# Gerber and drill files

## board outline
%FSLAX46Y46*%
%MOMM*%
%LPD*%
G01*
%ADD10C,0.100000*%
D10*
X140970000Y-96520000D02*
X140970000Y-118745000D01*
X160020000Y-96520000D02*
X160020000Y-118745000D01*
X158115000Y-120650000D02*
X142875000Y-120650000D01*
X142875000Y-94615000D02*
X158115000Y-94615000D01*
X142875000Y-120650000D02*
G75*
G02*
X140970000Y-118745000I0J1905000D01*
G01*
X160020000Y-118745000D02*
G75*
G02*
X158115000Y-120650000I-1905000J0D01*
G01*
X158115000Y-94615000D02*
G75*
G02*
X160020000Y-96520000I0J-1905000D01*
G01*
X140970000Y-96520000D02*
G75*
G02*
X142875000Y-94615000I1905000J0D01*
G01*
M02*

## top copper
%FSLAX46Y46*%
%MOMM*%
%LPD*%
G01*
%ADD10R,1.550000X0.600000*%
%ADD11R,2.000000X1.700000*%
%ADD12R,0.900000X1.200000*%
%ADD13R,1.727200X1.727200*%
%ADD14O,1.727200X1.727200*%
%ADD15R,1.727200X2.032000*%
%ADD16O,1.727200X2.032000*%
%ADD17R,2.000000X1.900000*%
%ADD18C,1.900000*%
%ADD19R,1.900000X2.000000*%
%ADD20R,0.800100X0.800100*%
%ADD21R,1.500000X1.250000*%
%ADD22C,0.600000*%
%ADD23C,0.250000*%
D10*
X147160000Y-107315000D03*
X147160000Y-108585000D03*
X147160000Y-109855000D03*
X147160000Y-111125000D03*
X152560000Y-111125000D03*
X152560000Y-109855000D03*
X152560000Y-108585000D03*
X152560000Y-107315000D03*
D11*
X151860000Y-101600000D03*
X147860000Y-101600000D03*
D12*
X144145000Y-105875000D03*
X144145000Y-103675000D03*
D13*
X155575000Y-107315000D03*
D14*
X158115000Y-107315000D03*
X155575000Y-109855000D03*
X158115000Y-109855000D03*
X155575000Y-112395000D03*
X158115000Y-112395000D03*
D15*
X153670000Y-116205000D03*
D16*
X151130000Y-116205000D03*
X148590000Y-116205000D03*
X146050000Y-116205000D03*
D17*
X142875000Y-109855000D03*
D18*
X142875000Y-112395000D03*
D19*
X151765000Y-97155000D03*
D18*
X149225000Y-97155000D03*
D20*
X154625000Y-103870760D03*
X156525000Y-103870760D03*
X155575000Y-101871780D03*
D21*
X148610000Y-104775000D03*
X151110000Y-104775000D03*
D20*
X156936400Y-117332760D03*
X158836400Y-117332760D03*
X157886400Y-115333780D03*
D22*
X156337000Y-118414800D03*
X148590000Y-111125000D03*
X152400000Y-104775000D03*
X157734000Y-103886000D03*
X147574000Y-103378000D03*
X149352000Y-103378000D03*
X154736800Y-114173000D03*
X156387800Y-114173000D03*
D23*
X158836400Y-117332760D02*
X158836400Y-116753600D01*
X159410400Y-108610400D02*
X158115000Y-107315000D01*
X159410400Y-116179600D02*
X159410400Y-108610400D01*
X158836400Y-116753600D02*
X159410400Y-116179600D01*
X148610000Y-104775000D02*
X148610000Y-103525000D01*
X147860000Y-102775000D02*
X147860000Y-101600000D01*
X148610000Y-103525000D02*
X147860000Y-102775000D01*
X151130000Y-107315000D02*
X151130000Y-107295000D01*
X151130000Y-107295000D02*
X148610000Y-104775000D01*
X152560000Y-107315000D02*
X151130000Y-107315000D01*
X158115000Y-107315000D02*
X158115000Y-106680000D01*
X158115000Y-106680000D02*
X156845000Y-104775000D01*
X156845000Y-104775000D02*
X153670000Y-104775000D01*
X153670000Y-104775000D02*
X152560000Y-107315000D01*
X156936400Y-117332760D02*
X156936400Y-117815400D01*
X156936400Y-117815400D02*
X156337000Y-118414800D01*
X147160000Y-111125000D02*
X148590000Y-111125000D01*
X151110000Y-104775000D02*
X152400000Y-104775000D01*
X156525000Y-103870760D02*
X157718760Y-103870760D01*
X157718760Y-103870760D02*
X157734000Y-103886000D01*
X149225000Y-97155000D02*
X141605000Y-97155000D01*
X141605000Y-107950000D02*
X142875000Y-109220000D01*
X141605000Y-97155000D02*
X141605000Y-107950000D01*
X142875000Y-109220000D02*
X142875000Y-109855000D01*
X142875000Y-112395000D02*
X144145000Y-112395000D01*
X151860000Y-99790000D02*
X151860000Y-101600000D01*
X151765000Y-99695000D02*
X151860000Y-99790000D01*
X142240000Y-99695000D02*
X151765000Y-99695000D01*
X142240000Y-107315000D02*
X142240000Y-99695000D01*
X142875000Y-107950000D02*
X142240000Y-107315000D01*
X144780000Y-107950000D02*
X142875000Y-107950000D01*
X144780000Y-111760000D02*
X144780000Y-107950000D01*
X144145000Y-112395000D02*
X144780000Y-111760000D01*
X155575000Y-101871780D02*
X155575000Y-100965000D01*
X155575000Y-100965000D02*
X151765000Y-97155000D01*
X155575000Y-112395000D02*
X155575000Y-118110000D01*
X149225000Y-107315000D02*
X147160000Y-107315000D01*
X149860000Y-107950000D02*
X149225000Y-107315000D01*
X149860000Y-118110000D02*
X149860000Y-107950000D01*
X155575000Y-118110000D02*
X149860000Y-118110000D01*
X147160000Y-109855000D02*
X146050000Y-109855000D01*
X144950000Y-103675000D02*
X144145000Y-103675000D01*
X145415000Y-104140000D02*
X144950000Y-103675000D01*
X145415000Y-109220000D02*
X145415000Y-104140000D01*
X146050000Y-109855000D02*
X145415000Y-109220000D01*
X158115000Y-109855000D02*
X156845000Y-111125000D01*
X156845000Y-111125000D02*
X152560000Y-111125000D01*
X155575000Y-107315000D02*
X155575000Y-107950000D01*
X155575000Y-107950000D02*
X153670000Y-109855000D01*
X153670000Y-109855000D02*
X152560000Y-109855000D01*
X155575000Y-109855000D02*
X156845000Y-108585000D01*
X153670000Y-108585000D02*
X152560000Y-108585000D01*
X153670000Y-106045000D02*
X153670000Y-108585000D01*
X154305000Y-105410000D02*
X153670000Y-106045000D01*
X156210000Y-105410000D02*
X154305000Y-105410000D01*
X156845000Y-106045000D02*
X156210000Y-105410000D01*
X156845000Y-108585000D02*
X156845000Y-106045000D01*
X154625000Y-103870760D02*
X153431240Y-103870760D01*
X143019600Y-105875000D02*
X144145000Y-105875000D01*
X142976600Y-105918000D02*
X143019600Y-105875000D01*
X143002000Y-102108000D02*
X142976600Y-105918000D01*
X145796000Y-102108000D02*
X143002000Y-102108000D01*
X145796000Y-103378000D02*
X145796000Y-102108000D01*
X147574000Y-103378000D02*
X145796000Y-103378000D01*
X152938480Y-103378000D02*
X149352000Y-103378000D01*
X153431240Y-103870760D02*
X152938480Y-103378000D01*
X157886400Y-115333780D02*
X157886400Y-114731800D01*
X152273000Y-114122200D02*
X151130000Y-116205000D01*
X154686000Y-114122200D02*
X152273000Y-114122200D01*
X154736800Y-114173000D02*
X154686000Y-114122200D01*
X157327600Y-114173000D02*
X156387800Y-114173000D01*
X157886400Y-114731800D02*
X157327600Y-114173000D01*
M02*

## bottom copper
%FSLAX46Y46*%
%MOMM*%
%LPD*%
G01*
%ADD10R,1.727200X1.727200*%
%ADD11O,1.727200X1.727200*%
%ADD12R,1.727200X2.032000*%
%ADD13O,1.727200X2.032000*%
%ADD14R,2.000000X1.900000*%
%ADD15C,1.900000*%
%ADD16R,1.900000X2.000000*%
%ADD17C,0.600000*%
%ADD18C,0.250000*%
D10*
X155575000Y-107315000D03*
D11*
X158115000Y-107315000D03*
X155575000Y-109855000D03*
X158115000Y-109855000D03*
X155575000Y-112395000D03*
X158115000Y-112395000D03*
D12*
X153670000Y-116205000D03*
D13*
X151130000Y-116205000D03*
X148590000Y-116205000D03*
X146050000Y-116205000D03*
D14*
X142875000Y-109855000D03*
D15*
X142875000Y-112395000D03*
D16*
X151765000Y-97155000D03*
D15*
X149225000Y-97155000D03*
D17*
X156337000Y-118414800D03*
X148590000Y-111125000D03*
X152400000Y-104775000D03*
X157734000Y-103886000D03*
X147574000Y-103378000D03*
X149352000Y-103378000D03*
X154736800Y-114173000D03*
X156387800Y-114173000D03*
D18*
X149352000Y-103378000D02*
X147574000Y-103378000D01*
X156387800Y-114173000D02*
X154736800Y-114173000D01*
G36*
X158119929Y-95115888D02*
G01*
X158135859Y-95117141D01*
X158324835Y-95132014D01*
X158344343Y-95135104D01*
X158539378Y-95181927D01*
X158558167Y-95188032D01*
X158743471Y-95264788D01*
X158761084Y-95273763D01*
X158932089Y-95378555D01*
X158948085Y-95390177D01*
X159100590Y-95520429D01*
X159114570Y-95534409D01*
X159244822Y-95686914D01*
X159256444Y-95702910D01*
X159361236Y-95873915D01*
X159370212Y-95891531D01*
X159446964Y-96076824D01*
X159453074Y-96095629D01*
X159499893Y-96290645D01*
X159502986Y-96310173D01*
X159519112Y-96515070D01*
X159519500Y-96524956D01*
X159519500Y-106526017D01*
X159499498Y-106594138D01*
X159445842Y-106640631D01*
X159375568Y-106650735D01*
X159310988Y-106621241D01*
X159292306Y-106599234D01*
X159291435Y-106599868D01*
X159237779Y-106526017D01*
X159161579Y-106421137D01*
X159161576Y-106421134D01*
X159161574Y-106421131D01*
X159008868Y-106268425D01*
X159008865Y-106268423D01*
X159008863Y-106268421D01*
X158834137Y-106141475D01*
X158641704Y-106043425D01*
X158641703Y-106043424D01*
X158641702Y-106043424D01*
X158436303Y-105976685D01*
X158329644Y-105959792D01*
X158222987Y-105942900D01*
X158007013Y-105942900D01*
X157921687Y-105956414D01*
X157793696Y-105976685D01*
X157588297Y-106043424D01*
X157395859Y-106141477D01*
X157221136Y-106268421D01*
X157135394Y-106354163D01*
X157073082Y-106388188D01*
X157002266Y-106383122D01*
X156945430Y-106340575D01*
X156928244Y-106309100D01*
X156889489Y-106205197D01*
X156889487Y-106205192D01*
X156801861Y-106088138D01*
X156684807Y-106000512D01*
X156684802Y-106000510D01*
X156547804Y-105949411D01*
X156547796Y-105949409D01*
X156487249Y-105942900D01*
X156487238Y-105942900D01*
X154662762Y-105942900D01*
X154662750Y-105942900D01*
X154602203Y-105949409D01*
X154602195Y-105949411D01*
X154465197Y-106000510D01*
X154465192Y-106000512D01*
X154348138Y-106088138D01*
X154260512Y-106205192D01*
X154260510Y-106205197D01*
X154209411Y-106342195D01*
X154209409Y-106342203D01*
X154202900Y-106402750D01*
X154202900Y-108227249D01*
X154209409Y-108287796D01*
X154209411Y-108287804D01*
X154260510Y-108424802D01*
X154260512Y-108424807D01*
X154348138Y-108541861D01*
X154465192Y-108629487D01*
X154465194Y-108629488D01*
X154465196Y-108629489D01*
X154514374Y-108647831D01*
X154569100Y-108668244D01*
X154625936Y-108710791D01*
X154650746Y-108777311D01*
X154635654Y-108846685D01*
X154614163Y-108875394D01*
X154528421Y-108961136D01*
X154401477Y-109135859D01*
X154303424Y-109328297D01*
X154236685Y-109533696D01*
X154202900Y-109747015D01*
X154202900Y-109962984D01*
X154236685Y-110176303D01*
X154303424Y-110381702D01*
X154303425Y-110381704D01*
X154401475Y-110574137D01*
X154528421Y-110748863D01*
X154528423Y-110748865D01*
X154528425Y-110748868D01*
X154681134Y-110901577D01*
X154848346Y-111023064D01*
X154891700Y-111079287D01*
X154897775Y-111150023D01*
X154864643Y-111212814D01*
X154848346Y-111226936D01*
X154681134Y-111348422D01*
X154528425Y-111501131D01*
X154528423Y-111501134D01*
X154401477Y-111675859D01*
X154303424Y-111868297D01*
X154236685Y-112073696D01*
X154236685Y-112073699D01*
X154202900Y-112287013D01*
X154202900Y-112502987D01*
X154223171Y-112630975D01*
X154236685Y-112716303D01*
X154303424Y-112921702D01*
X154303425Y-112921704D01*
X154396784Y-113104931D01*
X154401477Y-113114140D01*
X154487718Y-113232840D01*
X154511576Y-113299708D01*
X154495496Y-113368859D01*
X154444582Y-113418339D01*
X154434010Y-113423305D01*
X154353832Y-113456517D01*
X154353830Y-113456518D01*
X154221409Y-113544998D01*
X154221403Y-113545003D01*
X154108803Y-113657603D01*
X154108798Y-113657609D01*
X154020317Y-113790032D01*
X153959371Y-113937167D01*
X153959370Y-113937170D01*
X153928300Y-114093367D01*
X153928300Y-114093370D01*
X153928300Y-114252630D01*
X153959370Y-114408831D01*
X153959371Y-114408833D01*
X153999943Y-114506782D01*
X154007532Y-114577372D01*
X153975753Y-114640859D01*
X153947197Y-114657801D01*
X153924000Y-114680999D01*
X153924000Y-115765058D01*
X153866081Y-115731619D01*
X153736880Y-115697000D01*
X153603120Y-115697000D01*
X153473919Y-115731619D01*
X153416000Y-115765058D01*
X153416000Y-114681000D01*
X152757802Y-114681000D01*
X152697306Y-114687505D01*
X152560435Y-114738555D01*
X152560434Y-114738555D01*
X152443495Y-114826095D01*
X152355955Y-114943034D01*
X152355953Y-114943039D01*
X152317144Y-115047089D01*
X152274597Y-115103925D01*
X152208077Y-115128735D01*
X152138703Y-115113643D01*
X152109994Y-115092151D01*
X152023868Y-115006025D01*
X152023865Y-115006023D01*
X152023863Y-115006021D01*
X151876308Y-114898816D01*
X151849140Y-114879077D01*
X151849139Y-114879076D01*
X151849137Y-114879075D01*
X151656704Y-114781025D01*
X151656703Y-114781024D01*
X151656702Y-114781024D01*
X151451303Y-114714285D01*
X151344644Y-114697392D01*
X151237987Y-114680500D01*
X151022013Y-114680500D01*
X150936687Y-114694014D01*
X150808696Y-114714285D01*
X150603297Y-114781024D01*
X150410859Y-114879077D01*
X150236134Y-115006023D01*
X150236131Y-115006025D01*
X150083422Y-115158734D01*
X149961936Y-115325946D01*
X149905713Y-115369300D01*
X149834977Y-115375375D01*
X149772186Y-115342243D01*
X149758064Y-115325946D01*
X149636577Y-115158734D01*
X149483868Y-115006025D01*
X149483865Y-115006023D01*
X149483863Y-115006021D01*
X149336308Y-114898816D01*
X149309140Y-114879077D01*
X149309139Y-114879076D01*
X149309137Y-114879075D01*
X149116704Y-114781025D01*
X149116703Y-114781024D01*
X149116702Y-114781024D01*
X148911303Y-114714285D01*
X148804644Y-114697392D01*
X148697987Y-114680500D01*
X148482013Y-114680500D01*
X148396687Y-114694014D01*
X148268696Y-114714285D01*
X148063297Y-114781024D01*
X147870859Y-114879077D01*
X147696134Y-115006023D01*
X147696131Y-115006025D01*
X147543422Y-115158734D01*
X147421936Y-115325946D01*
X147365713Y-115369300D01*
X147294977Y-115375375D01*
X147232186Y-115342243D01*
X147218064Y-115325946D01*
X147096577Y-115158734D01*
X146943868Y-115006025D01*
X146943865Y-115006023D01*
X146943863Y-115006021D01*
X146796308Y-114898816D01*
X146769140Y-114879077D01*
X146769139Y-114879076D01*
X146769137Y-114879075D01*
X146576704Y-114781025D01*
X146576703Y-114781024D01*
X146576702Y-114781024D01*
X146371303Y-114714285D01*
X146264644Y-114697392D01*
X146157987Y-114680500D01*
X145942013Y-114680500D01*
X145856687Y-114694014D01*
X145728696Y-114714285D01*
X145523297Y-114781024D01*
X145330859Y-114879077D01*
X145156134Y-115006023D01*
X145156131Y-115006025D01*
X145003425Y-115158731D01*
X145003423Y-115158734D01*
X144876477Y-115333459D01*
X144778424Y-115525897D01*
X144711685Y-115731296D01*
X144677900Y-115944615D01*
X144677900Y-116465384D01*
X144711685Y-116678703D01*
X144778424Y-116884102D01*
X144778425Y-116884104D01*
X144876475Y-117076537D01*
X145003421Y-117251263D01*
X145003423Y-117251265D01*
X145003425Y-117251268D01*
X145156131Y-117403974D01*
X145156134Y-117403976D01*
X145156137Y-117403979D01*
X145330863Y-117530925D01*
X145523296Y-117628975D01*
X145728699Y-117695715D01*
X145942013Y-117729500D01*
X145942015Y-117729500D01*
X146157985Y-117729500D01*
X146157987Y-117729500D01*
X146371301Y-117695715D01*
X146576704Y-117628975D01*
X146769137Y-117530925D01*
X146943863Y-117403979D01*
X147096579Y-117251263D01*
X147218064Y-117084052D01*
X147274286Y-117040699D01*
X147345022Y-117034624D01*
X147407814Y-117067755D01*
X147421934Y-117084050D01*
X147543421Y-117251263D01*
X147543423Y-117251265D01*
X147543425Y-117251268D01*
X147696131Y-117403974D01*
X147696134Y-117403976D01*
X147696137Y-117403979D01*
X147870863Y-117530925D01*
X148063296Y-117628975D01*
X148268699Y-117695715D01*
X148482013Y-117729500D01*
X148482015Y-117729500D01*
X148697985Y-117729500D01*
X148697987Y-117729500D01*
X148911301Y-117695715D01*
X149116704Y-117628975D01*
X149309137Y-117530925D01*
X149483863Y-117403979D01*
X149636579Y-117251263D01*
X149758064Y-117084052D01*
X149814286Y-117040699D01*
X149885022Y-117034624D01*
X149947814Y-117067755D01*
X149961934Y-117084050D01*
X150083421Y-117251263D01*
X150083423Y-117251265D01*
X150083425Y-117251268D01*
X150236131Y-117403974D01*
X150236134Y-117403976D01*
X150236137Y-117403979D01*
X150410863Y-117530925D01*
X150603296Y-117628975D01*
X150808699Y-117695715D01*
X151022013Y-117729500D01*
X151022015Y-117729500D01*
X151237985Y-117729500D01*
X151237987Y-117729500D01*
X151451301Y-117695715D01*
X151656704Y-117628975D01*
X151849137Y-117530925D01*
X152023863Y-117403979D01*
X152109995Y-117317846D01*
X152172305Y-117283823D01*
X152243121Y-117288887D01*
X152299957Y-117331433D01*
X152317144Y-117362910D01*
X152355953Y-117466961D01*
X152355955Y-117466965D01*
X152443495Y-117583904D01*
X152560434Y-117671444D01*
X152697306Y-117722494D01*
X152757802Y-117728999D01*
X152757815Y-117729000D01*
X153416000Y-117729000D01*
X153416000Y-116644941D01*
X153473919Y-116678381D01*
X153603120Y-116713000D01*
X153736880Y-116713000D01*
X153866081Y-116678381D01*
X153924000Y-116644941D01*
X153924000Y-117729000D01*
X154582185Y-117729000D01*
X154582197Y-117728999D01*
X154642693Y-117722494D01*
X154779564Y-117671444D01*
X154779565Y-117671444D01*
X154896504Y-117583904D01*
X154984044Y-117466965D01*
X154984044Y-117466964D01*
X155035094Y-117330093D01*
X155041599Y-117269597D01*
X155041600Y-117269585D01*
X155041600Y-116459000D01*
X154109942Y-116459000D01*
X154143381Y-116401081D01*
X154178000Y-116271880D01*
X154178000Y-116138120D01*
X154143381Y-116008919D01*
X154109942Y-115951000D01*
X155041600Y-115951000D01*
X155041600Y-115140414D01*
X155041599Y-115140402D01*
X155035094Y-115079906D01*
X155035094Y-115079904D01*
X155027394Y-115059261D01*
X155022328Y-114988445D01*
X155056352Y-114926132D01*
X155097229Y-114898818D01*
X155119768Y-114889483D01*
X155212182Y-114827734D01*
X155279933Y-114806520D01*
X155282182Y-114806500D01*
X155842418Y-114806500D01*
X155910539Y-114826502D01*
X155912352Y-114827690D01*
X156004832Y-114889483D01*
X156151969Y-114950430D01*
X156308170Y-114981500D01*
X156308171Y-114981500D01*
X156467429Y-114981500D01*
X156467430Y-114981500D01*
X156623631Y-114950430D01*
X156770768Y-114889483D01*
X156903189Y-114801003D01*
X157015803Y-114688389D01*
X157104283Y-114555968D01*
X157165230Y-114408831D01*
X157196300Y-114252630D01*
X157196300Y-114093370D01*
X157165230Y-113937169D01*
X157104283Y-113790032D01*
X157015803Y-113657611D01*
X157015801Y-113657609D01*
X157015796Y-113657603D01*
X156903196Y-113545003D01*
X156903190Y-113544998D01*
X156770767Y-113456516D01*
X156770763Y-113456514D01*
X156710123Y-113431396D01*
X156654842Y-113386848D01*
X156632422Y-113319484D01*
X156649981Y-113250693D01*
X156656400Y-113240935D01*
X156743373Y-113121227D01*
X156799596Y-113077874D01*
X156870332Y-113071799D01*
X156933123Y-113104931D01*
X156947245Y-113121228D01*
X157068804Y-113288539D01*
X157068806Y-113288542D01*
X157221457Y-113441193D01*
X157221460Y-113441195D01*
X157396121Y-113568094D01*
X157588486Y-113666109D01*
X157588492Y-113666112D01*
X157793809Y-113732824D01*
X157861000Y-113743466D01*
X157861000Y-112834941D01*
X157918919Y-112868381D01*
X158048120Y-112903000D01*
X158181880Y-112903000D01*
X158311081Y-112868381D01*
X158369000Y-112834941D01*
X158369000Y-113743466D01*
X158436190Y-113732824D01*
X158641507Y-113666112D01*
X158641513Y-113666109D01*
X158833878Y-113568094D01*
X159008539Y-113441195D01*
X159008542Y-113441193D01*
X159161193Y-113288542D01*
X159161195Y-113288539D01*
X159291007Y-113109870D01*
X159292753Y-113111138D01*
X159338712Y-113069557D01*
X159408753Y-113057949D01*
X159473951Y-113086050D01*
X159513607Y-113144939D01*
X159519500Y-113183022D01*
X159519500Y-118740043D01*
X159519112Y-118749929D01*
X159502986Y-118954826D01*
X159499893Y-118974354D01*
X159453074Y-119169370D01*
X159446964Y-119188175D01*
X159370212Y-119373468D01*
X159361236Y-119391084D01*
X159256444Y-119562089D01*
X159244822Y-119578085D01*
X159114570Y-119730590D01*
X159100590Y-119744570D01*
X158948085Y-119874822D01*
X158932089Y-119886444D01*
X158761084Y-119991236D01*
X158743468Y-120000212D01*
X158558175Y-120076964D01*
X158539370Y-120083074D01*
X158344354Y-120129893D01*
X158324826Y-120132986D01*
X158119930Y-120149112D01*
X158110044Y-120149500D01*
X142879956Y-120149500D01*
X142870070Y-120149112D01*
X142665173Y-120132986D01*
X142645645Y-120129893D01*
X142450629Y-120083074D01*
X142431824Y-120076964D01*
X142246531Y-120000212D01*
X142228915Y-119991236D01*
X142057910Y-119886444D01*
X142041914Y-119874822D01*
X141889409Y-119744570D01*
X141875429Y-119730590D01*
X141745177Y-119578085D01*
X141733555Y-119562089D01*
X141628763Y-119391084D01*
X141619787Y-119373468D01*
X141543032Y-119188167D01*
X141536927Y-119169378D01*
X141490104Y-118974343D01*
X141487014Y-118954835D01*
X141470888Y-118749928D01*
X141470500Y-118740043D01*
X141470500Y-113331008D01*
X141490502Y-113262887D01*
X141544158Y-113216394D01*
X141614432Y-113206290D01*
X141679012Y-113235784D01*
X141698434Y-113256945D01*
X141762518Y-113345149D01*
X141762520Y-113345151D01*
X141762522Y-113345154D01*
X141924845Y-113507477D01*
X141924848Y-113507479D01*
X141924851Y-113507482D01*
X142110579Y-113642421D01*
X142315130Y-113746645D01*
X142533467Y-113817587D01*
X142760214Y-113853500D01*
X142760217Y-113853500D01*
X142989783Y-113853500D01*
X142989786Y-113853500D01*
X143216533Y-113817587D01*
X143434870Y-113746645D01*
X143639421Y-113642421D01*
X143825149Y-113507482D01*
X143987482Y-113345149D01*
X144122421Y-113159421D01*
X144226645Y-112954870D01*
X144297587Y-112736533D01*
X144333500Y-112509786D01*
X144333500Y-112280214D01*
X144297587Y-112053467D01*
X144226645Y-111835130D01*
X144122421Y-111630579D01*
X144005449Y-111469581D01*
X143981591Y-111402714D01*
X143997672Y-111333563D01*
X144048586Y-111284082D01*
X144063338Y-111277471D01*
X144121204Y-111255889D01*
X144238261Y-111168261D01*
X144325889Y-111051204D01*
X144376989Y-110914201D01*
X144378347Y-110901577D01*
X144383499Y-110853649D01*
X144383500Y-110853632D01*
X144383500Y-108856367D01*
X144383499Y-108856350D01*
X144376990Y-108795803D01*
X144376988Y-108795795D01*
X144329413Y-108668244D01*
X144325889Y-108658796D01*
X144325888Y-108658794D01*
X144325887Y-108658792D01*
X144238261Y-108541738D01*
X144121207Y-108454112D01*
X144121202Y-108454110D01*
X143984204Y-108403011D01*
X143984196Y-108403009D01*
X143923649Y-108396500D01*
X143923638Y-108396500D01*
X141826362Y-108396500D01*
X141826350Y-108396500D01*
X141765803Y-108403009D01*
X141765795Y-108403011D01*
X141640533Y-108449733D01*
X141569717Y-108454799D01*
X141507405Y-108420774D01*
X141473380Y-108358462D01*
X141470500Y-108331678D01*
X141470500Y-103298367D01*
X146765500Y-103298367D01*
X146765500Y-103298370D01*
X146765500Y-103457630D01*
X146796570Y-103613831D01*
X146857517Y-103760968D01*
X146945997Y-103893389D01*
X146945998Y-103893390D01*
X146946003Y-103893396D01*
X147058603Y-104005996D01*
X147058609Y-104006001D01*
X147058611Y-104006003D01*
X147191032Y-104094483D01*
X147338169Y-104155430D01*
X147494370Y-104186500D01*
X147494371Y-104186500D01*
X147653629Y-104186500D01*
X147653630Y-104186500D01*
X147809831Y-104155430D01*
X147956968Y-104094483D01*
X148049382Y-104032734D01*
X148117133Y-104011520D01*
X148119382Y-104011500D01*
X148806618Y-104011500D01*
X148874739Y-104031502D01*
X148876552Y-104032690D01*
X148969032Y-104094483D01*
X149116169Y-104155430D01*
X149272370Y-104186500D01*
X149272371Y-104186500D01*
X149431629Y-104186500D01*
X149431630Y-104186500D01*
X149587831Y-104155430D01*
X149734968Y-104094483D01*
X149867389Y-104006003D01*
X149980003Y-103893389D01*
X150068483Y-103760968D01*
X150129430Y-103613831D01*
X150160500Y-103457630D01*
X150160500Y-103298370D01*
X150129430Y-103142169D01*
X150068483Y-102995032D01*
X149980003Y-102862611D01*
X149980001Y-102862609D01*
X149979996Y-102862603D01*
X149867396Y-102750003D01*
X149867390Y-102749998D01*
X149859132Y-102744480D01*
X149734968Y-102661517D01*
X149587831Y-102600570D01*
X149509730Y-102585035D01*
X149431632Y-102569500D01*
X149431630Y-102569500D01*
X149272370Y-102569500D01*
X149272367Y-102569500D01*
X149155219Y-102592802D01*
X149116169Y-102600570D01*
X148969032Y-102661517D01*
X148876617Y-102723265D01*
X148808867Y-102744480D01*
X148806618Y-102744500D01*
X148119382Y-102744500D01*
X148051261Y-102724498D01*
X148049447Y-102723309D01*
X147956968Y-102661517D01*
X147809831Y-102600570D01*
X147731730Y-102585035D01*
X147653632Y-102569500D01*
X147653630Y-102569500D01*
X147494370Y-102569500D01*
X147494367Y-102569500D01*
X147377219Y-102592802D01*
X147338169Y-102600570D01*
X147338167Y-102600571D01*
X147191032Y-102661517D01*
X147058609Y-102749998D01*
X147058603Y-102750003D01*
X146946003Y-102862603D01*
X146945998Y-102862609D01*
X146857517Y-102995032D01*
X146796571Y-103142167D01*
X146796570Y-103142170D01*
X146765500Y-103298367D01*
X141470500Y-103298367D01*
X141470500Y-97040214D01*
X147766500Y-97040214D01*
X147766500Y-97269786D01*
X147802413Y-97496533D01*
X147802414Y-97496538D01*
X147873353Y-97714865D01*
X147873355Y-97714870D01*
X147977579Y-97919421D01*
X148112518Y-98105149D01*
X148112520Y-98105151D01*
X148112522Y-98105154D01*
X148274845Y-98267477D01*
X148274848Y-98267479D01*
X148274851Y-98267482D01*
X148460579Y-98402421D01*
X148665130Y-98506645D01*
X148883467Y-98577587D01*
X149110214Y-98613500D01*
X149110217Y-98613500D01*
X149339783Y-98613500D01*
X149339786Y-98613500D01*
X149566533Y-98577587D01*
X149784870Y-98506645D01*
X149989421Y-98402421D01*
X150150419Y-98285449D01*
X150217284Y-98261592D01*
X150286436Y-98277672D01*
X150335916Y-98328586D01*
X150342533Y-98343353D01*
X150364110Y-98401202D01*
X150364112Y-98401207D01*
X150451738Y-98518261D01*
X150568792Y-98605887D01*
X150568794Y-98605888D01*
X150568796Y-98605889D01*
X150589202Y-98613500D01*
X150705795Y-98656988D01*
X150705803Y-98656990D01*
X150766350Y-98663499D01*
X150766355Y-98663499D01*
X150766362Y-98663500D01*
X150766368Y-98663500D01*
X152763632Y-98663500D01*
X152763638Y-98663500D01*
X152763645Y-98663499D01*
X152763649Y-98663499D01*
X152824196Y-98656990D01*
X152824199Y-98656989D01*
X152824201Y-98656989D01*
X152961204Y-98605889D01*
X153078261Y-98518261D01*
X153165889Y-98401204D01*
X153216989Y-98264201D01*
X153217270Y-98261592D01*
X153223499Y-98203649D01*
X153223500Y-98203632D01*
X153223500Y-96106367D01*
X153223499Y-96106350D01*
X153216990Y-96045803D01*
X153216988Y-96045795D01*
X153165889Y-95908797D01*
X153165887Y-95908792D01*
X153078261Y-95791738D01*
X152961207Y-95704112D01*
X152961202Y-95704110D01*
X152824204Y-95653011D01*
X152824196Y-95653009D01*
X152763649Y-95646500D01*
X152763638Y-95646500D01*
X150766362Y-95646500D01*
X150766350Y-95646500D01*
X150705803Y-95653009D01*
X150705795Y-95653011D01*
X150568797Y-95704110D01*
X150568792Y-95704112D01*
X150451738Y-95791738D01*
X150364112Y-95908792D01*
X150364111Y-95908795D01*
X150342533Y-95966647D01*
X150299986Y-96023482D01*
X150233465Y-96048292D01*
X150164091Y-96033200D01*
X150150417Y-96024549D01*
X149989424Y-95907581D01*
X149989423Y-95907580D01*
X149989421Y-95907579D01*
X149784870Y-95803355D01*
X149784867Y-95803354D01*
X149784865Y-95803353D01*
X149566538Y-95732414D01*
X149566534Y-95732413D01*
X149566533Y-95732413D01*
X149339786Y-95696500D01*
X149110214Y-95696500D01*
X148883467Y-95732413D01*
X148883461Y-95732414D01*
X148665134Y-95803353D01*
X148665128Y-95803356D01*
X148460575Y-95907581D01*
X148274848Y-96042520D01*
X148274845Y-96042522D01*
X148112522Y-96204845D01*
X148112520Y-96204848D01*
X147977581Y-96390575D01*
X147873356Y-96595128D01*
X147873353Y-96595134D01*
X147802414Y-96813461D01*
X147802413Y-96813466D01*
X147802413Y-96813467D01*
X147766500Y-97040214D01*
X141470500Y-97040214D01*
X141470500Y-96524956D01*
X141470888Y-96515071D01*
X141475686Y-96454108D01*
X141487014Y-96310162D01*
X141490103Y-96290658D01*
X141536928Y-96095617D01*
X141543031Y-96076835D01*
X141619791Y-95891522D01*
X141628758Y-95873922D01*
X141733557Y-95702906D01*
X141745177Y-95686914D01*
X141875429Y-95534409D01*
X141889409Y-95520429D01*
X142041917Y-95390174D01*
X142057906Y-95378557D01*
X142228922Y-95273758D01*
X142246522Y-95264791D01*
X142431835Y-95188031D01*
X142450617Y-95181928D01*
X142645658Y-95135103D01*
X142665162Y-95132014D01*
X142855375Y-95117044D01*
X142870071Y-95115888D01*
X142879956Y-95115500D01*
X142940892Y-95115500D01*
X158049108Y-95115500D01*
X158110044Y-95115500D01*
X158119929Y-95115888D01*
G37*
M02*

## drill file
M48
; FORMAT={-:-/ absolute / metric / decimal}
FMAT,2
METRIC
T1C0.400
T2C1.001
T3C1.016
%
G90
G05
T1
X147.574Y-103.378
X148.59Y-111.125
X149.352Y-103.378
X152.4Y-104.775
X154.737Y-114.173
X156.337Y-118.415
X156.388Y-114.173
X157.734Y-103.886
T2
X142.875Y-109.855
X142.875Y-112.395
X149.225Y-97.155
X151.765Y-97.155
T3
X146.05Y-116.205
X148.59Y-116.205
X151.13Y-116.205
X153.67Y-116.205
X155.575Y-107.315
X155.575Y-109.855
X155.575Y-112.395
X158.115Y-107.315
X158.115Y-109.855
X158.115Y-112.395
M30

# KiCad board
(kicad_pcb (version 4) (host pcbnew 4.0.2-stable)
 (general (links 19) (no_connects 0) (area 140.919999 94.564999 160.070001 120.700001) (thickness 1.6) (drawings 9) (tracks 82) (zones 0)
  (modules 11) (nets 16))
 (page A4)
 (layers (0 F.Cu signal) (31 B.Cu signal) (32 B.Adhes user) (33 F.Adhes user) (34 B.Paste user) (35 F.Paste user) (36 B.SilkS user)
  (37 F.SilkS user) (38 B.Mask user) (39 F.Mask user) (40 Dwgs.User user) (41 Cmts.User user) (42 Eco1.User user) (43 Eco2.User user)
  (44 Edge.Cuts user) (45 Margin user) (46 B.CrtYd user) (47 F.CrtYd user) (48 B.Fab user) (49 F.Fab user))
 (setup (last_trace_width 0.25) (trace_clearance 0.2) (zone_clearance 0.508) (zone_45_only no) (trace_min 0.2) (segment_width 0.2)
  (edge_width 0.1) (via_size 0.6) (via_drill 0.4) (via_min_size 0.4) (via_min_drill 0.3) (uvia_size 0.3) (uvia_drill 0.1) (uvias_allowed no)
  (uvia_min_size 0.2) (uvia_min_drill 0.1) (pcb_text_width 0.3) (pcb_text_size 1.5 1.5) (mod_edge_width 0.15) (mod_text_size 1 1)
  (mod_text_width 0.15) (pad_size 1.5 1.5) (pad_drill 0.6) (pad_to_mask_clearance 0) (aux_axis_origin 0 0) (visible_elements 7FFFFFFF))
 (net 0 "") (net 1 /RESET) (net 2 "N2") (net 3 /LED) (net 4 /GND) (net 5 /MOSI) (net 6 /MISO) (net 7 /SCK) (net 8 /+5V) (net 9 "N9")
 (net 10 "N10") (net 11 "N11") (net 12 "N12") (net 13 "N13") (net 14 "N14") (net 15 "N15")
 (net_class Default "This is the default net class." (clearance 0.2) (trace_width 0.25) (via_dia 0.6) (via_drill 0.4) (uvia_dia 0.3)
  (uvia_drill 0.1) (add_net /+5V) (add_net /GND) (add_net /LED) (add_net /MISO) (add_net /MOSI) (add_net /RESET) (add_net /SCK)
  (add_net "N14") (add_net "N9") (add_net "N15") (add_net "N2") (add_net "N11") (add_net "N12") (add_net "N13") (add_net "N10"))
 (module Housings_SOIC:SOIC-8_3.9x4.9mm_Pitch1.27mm (layer F.Cu) (at 149.86 109.22)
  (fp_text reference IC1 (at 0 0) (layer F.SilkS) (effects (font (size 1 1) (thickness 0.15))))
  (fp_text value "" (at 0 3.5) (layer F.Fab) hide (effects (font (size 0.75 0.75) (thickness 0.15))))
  (pad 1 smd rect (at -2.7 -1.905) (size 1.55 0.6) (layers F.Cu F.Paste F.Mask) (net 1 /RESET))
  (pad 2 smd rect (at -2.7 -0.635) (size 1.55 0.6) (layers F.Cu F.Paste F.Mask) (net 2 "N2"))
  (pad 3 smd rect (at -2.7 0.635) (size 1.55 0.6) (layers F.Cu F.Paste F.Mask) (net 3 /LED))
  (pad 4 smd rect (at -2.7 1.905) (size 1.55 0.6) (layers F.Cu F.Paste F.Mask) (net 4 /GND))
  (pad 5 smd rect (at 2.7 1.905) (size 1.55 0.6) (layers F.Cu F.Paste F.Mask) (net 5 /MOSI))
  (pad 6 smd rect (at 2.7 0.635) (size 1.55 0.6) (layers F.Cu F.Paste F.Mask) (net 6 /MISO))
  (pad 7 smd rect (at 2.7 -0.635) (size 1.55 0.6) (layers F.Cu F.Paste F.Mask) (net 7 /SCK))
  (pad 8 smd rect (at 2.7 -1.905) (size 1.55 0.6) (layers F.Cu F.Paste F.Mask) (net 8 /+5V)))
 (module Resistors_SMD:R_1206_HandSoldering (layer F.Cu) (at 149.86 101.6 180)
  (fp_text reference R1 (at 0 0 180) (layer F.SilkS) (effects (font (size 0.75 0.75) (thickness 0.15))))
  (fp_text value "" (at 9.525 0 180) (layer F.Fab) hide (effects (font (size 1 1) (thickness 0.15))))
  (pad 1 smd rect (at -2 0 180) (size 2 1.7) (layers F.Cu F.Paste F.Mask) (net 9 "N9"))
  (pad 2 smd rect (at 2 0 180) (size 2 1.7) (layers F.Cu F.Paste F.Mask) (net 8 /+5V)))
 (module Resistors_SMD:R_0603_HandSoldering (layer F.Cu) (at 144.145 104.775 90)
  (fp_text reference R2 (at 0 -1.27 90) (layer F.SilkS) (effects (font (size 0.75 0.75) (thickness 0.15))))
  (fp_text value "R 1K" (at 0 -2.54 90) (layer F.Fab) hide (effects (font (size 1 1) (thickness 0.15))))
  (pad 1 smd rect (at -1.1 0 90) (size 1.2 0.9) (layers F.Cu F.Paste F.Mask) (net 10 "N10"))
  (pad 2 smd rect (at 1.1 0 90) (size 1.2 0.9) (layers F.Cu F.Paste F.Mask) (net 3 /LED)))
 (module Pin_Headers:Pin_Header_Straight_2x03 (layer F.Cu) (at 155.575 107.315)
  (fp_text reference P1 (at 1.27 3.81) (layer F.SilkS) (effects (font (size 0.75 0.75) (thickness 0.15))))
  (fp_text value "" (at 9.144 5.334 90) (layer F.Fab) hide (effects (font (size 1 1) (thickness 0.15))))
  (pad 1 thru_hole rect (at 0 0) (size 1.7272 1.7272) (drill 1.016) (layers *.Cu *.Mask F.SilkS) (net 6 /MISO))
  (pad 2 thru_hole oval (at 2.54 0) (size 1.7272 1.7272) (drill 1.016) (layers *.Cu *.Mask F.SilkS) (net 8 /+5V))
  (pad 3 thru_hole oval (at 0 2.54) (size 1.7272 1.7272) (drill 1.016) (layers *.Cu *.Mask F.SilkS) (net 7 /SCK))
  (pad 4 thru_hole oval (at 2.54 2.54) (size 1.7272 1.7272) (drill 1.016) (layers *.Cu *.Mask F.SilkS) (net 5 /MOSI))
  (pad 5 thru_hole oval (at 0 5.08) (size 1.7272 1.7272) (drill 1.016) (layers *.Cu *.Mask F.SilkS) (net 1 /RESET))
  (pad 6 thru_hole oval (at 2.54 5.08) (size 1.7272 1.7272) (drill 1.016) (layers *.Cu *.Mask F.SilkS) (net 4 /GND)))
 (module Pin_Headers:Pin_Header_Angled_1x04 (layer F.Cu) (at 153.67 116.205 270)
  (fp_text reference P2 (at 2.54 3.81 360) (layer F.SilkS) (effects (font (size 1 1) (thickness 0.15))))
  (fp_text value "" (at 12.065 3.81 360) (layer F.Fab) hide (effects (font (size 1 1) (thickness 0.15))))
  (pad 1 thru_hole rect (at 0 0 270) (size 2.032 1.7272) (drill 1.016) (layers *.Cu *.Mask F.SilkS) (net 4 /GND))
  (pad 2 thru_hole oval (at 0 2.54 270) (size 2.032 1.7272) (drill 1.016) (layers *.Cu *.Mask F.SilkS) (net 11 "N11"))
  (pad 3 thru_hole oval (at 0 5.08 270) (size 2.032 1.7272) (drill 1.016) (layers *.Cu *.Mask F.SilkS) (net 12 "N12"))
  (pad 4 thru_hole oval (at 0 7.62 270) (size 2.032 1.7272) (drill 1.016) (layers *.Cu *.Mask F.SilkS) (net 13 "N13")))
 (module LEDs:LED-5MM (layer F.Cu) (at 142.875 109.855 270)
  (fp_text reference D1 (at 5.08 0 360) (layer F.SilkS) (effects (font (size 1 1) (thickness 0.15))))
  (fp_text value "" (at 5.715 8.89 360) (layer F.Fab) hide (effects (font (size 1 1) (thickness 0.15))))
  (pad 1 thru_hole rect (at 0 0) (size 2 1.9) (drill 1.00076) (layers *.Cu *.Mask F.SilkS) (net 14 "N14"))
  (pad 2 thru_hole circle (at 2.54 0 270) (size 1.9 1.9) (drill 1.00076) (layers *.Cu *.Mask F.SilkS) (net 9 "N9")))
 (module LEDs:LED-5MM (layer F.Cu) (at 151.765 97.155 180)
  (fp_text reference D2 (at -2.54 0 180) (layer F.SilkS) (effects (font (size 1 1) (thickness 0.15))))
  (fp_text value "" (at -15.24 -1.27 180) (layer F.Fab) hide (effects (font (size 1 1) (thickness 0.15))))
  (pad 1 thru_hole rect (at 0 0 270) (size 2 1.9) (drill 1.00076) (layers *.Cu *.Mask F.SilkS) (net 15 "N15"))
  (pad 2 thru_hole circle (at 2.54 0 180) (size 1.9 1.9) (drill 1.00076) (layers *.Cu *.Mask F.SilkS) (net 14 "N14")))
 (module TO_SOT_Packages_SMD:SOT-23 (layer F.Cu) (at 155.575 102.87)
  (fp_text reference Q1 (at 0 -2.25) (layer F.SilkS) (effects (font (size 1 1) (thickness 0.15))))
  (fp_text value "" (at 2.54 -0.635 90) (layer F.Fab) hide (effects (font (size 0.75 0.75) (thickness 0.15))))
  (pad 1 smd rect (at -0.95 1.00076) (size 0.8001 0.8001) (layers F.Cu F.Paste F.Mask) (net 10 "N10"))
  (pad 2 smd rect (at 0.95 1.00076) (size 0.8001 0.8001) (layers F.Cu F.Paste F.Mask) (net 4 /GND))
  (pad 3 smd rect (at 0 -0.99822) (size 0.8001 0.8001) (layers F.Cu F.Paste F.Mask) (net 15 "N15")))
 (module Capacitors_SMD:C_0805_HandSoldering (layer F.Cu) (at 149.86 104.775)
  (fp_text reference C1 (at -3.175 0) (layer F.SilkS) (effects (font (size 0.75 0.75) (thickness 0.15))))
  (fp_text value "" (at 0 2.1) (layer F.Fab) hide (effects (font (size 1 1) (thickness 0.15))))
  (pad 1 smd rect (at -1.25 0) (size 1.5 1.25) (layers F.Cu F.Paste F.Mask) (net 8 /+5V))
  (pad 2 smd rect (at 1.25 0) (size 1.5 1.25) (layers F.Cu F.Paste F.Mask) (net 4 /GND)))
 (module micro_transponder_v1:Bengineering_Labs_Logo (layer B.Cu) (at 151.3332 106.6292 270)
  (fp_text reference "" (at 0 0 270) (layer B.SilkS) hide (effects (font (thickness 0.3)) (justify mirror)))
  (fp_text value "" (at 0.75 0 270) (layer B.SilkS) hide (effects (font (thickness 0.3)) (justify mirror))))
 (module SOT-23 (layer F.Cu) (at 157.8864 116.332)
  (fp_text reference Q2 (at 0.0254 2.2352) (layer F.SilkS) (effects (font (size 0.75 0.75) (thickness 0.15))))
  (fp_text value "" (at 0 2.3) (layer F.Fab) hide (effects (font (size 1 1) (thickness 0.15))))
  (pad 1 smd rect (at -0.95 1.00076) (size 0.8001 0.8001) (layers F.Cu F.Paste F.Mask) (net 4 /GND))
  (pad 2 smd rect (at 0.95 1.00076) (size 0.8001 0.8001) (layers F.Cu F.Paste F.Mask) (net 8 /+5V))
  (pad 3 smd rect (at 0 -0.99822) (size 0.8001 0.8001) (layers F.Cu F.Paste F.Mask) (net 11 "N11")))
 (gr_line (start 140.97 96.52) (end 140.97 118.745) (angle 90) (layer Edge.Cuts) (width 0.1))
 (gr_line (start 160.02 96.52) (end 160.02 118.745) (angle 90) (layer Edge.Cuts) (width 0.1))
 (gr_line (start 158.115 120.65) (end 142.875 120.65) (angle 90) (layer Edge.Cuts) (width 0.1))
 (gr_line (start 142.875 94.615) (end 158.115 94.615) (angle 90) (layer Edge.Cuts) (width 0.1))
 (gr_arc (start 142.875 118.745) (end 142.875 120.65) (angle 90) (layer Edge.Cuts) (width 0.1))
 (gr_arc (start 158.115 118.745) (end 160.02 118.745) (angle 90) (layer Edge.Cuts) (width 0.1))
 (gr_arc (start 158.115 96.52) (end 158.115 94.615) (angle 90) (layer Edge.Cuts) (width 0.1))
 (gr_arc (start 142.875 96.52) (end 140.97 96.52) (angle 90) (layer Edge.Cuts) (width 0.1))
 (segment (start 158.8364 117.33276) (end 158.8364 116.7536) (width 0.25) (layer F.Cu) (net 8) (status 10))
 (segment (start 159.4104 108.6104) (end 158.115 107.315) (width 0.25) (layer F.Cu) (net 8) (status 20))
 (segment (start 159.4104 116.1796) (end 159.4104 108.6104) (width 0.25) (layer F.Cu) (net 8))
 (segment (start 158.8364 116.7536) (end 159.4104 116.1796) (width 0.25) (layer F.Cu) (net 8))
 (segment (start 148.61 104.775) (end 148.61 103.525) (width 0.25) (layer F.Cu) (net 8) (status 10))
 (segment (start 147.86 102.775) (end 147.86 101.6) (width 0.25) (layer F.Cu) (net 8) (status 20))
 (segment (start 148.61 103.525) (end 147.86 102.775) (width 0.25) (layer F.Cu) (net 8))
 (segment (start 151.13 107.315) (end 151.13 107.295) (width 0.25) (layer F.Cu) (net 8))
 (segment (start 151.13 107.295) (end 148.61 104.775) (width 0.25) (layer F.Cu) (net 8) (status 20))
 (segment (start 152.56 107.315) (end 151.13 107.315) (width 0.25) (layer F.Cu) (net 8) (status 10))
 (segment (start 158.115 107.315) (end 158.115 106.68) (width 0.25) (layer F.Cu) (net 8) (status 30))
 (segment (start 158.115 106.68) (end 156.845 104.775) (width 0.25) (layer F.Cu) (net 8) (status 10))
 (segment (start 156.845 104.775) (end 153.67 104.775) (width 0.25) (layer F.Cu) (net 8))
 (segment (start 153.67 104.775) (end 152.56 107.315) (width 0.25) (layer F.Cu) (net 8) (status 20))
 (segment (start 156.9364 117.33276) (end 156.9364 117.8154) (width 0.25) (layer F.Cu) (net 4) (status 10))
 (via (at 156.337 118.4148) (size 0.6) (drill 0.4) (layers F.Cu B.Cu) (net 4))
 (segment (start 156.9364 117.8154) (end 156.337 118.4148) (width 0.25) (layer F.Cu) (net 4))
 (segment (start 147.16 111.125) (end 148.59 111.125) (width 0.25) (layer F.Cu) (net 4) (status 10))
 (via (at 148.59 111.125) (size 0.6) (drill 0.4) (layers F.Cu B.Cu) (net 4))
 (segment (start 151.11 104.775) (end 152.4 104.775) (width 0.25) (layer F.Cu) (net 4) (status 10))
 (via (at 152.4 104.775) (size 0.6) (drill 0.4) (layers F.Cu B.Cu) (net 4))
 (segment (start 156.525 103.87076) (end 157.71876 103.87076) (width 0.25) (layer F.Cu) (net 4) (status 10))
 (via (at 157.734 103.886) (size 0.6) (drill 0.4) (layers F.Cu B.Cu) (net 4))
 (segment (start 157.71876 103.87076) (end 157.734 103.886) (width 0.25) (layer F.Cu) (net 4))
 (segment (start 149.225 97.155) (end 141.605 97.155) (width 0.25) (layer F.Cu) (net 14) (status 10))
 (segment (start 141.605 107.95) (end 142.875 109.22) (width 0.25) (layer F.Cu) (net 14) (status 20))
 (segment (start 141.605 97.155) (end 141.605 107.95) (width 0.25) (layer F.Cu) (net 14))
 (segment (start 142.875 109.22) (end 142.875 109.855) (width 0.25) (layer F.Cu) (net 14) (status 30))
 (segment (start 142.875 112.395) (end 144.145 112.395) (width 0.25) (layer F.Cu) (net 9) (status 10))
 (segment (start 151.86 99.79) (end 151.86 101.6) (width 0.25) (layer F.Cu) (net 9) (status 20))
 (segment (start 151.765 99.695) (end 151.86 99.79) (width 0.25) (layer F.Cu) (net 9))
 (segment (start 142.24 99.695) (end 151.765 99.695) (width 0.25) (layer F.Cu) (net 9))
 (segment (start 142.24 107.315) (end 142.24 99.695) (width 0.25) (layer F.Cu) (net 9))
 (segment (start 142.875 107.95) (end 142.24 107.315) (width 0.25) (layer F.Cu) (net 9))
 (segment (start 144.78 107.95) (end 142.875 107.95) (width 0.25) (layer F.Cu) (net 9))
 (segment (start 144.78 111.76) (end 144.78 107.95) (width 0.25) (layer F.Cu) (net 9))
 (segment (start 144.145 112.395) (end 144.78 111.76) (width 0.25) (layer F.Cu) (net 9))
 (segment (start 155.575 101.87178) (end 155.575 100.965) (width 0.25) (layer F.Cu) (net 15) (status 10))
 (segment (start 155.575 100.965) (end 151.765 97.155) (width 0.25) (layer F.Cu) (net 15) (status 20))
 (segment (start 155.575 112.395) (end 155.575 118.11) (width 0.25) (layer F.Cu) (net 1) (status 10))
 (segment (start 149.225 107.315) (end 147.16 107.315) (width 0.25) (layer F.Cu) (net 1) (status 20))
 (segment (start 149.86 107.95) (end 149.225 107.315) (width 0.25) (layer F.Cu) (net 1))
 (segment (start 149.86 118.11) (end 149.86 107.95) (width 0.25) (layer F.Cu) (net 1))
 (segment (start 155.575 118.11) (end 149.86 118.11) (width 0.25) (layer F.Cu) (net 1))
 (segment (start 147.16 109.855) (end 146.05 109.855) (width 0.25) (layer F.Cu) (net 3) (status 10))
 (segment (start 144.95 103.675) (end 144.145 103.675) (width 0.25) (layer F.Cu) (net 3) (status 20))
 (segment (start 145.415 104.14) (end 144.95 103.675) (width 0.25) (layer F.Cu) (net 3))
 (segment (start 145.415 109.22) (end 145.415 104.14) (width 0.25) (layer F.Cu) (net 3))
 (segment (start 146.05 109.855) (end 145.415 109.22) (width 0.25) (layer F.Cu) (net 3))
 (segment (start 158.115 109.855) (end 156.845 111.125) (width 0.25) (layer F.Cu) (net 5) (status 10))
 (segment (start 156.845 111.125) (end 152.56 111.125) (width 0.25) (layer F.Cu) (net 5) (status 20))
 (segment (start 155.575 107.315) (end 155.575 107.95) (width 0.25) (layer F.Cu) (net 6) (status 30))
 (segment (start 155.575 107.95) (end 153.67 109.855) (width 0.25) (layer F.Cu) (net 6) (status 10))
 (segment (start 153.67 109.855) (end 152.56 109.855) (width 0.25) (layer F.Cu) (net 6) (status 20))
 (segment (start 155.575 109.855) (end 156.845 108.585) (width 0.25) (layer F.Cu) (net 7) (status 10))
 (segment (start 153.67 108.585) (end 152.56 108.585) (width 0.25) (layer F.Cu) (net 7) (status 20))
 (segment (start 153.67 106.045) (end 153.67 108.585) (width 0.25) (layer F.Cu) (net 7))
 (segment (start 154.305 105.41) (end 153.67 106.045) (width 0.25) (layer F.Cu) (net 7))
 (segment (start 156.21 105.41) (end 154.305 105.41) (width 0.25) (layer F.Cu) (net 7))
 (segment (start 156.845 106.045) (end 156.21 105.41) (width 0.25) (layer F.Cu) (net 7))
 (segment (start 156.845 108.585) (end 156.845 106.045) (width 0.25) (layer F.Cu) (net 7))
 (segment (start 154.625 103.87076) (end 153.43124 103.87076) (width 0.25) (layer F.Cu) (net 10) (status 10))
 (segment (start 143.0196 105.875) (end 144.145 105.875) (width 0.25) (layer F.Cu) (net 10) (status 20))
 (segment (start 142.9766 105.918) (end 143.0196 105.875) (width 0.25) (layer F.Cu) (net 10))
 (segment (start 143.002 102.108) (end 142.9766 105.918) (width 0.25) (layer F.Cu) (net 10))
 (segment (start 145.796 102.108) (end 143.002 102.108) (width 0.25) (layer F.Cu) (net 10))
 (segment (start 145.796 103.378) (end 145.796 102.108) (width 0.25) (layer F.Cu) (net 10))
 (segment (start 147.574 103.378) (end 145.796 103.378) (width 0.25) (layer F.Cu) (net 10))
 (via (at 147.574 103.378) (size 0.6) (drill 0.4) (layers F.Cu B.Cu) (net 10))
 (segment (start 149.352 103.378) (end 147.574 103.378) (width 0.25) (layer B.Cu) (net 10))
 (via (at 149.352 103.378) (size 0.6) (drill 0.4) (layers F.Cu B.Cu) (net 10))
 (segment (start 152.93848 103.378) (end 149.352 103.378) (width 0.25) (layer F.Cu) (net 10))
 (segment (start 153.43124 103.87076) (end 152.93848 103.378) (width 0.25) (layer F.Cu) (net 10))
 (segment (start 157.8864 115.33378) (end 157.8864 114.7318) (width 0.25) (layer F.Cu) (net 11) (status 10))
 (segment (start 152.273 114.1222) (end 151.13 116.205) (width 0.25) (layer F.Cu) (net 11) (status 20))
 (segment (start 154.686 114.1222) (end 152.273 114.1222) (width 0.25) (layer F.Cu) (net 11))
 (segment (start 154.7368 114.173) (end 154.686 114.1222) (width 0.25) (layer F.Cu) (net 11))
 (via (at 154.7368 114.173) (size 0.6) (drill 0.4) (layers F.Cu B.Cu) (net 11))
 (segment (start 156.3878 114.173) (end 154.7368 114.173) (width 0.25) (layer B.Cu) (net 11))
 (via (at 156.3878 114.173) (size 0.6) (drill 0.4) (layers F.Cu B.Cu) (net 11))
 (segment (start 157.3276 114.173) (end 156.3878 114.173) (width 0.25) (layer F.Cu) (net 11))
 (segment (start 157.8864 114.7318) (end 157.3276 114.173) (width 0.25) (layer F.Cu) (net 11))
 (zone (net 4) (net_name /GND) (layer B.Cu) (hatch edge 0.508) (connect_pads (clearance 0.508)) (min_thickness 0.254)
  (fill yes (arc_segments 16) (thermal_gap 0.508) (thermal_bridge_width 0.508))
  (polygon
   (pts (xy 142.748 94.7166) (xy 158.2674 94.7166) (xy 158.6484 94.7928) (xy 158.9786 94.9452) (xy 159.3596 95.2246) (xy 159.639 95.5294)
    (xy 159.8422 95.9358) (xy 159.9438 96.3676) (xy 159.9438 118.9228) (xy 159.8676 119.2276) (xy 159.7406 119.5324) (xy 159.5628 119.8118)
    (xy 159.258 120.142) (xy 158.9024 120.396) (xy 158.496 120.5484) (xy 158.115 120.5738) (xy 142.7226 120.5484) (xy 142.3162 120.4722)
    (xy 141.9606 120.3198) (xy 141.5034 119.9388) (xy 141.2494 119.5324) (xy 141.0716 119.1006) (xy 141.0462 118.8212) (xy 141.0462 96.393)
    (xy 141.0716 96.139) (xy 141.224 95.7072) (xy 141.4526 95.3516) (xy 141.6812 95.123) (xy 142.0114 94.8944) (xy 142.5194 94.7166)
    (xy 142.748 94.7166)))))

